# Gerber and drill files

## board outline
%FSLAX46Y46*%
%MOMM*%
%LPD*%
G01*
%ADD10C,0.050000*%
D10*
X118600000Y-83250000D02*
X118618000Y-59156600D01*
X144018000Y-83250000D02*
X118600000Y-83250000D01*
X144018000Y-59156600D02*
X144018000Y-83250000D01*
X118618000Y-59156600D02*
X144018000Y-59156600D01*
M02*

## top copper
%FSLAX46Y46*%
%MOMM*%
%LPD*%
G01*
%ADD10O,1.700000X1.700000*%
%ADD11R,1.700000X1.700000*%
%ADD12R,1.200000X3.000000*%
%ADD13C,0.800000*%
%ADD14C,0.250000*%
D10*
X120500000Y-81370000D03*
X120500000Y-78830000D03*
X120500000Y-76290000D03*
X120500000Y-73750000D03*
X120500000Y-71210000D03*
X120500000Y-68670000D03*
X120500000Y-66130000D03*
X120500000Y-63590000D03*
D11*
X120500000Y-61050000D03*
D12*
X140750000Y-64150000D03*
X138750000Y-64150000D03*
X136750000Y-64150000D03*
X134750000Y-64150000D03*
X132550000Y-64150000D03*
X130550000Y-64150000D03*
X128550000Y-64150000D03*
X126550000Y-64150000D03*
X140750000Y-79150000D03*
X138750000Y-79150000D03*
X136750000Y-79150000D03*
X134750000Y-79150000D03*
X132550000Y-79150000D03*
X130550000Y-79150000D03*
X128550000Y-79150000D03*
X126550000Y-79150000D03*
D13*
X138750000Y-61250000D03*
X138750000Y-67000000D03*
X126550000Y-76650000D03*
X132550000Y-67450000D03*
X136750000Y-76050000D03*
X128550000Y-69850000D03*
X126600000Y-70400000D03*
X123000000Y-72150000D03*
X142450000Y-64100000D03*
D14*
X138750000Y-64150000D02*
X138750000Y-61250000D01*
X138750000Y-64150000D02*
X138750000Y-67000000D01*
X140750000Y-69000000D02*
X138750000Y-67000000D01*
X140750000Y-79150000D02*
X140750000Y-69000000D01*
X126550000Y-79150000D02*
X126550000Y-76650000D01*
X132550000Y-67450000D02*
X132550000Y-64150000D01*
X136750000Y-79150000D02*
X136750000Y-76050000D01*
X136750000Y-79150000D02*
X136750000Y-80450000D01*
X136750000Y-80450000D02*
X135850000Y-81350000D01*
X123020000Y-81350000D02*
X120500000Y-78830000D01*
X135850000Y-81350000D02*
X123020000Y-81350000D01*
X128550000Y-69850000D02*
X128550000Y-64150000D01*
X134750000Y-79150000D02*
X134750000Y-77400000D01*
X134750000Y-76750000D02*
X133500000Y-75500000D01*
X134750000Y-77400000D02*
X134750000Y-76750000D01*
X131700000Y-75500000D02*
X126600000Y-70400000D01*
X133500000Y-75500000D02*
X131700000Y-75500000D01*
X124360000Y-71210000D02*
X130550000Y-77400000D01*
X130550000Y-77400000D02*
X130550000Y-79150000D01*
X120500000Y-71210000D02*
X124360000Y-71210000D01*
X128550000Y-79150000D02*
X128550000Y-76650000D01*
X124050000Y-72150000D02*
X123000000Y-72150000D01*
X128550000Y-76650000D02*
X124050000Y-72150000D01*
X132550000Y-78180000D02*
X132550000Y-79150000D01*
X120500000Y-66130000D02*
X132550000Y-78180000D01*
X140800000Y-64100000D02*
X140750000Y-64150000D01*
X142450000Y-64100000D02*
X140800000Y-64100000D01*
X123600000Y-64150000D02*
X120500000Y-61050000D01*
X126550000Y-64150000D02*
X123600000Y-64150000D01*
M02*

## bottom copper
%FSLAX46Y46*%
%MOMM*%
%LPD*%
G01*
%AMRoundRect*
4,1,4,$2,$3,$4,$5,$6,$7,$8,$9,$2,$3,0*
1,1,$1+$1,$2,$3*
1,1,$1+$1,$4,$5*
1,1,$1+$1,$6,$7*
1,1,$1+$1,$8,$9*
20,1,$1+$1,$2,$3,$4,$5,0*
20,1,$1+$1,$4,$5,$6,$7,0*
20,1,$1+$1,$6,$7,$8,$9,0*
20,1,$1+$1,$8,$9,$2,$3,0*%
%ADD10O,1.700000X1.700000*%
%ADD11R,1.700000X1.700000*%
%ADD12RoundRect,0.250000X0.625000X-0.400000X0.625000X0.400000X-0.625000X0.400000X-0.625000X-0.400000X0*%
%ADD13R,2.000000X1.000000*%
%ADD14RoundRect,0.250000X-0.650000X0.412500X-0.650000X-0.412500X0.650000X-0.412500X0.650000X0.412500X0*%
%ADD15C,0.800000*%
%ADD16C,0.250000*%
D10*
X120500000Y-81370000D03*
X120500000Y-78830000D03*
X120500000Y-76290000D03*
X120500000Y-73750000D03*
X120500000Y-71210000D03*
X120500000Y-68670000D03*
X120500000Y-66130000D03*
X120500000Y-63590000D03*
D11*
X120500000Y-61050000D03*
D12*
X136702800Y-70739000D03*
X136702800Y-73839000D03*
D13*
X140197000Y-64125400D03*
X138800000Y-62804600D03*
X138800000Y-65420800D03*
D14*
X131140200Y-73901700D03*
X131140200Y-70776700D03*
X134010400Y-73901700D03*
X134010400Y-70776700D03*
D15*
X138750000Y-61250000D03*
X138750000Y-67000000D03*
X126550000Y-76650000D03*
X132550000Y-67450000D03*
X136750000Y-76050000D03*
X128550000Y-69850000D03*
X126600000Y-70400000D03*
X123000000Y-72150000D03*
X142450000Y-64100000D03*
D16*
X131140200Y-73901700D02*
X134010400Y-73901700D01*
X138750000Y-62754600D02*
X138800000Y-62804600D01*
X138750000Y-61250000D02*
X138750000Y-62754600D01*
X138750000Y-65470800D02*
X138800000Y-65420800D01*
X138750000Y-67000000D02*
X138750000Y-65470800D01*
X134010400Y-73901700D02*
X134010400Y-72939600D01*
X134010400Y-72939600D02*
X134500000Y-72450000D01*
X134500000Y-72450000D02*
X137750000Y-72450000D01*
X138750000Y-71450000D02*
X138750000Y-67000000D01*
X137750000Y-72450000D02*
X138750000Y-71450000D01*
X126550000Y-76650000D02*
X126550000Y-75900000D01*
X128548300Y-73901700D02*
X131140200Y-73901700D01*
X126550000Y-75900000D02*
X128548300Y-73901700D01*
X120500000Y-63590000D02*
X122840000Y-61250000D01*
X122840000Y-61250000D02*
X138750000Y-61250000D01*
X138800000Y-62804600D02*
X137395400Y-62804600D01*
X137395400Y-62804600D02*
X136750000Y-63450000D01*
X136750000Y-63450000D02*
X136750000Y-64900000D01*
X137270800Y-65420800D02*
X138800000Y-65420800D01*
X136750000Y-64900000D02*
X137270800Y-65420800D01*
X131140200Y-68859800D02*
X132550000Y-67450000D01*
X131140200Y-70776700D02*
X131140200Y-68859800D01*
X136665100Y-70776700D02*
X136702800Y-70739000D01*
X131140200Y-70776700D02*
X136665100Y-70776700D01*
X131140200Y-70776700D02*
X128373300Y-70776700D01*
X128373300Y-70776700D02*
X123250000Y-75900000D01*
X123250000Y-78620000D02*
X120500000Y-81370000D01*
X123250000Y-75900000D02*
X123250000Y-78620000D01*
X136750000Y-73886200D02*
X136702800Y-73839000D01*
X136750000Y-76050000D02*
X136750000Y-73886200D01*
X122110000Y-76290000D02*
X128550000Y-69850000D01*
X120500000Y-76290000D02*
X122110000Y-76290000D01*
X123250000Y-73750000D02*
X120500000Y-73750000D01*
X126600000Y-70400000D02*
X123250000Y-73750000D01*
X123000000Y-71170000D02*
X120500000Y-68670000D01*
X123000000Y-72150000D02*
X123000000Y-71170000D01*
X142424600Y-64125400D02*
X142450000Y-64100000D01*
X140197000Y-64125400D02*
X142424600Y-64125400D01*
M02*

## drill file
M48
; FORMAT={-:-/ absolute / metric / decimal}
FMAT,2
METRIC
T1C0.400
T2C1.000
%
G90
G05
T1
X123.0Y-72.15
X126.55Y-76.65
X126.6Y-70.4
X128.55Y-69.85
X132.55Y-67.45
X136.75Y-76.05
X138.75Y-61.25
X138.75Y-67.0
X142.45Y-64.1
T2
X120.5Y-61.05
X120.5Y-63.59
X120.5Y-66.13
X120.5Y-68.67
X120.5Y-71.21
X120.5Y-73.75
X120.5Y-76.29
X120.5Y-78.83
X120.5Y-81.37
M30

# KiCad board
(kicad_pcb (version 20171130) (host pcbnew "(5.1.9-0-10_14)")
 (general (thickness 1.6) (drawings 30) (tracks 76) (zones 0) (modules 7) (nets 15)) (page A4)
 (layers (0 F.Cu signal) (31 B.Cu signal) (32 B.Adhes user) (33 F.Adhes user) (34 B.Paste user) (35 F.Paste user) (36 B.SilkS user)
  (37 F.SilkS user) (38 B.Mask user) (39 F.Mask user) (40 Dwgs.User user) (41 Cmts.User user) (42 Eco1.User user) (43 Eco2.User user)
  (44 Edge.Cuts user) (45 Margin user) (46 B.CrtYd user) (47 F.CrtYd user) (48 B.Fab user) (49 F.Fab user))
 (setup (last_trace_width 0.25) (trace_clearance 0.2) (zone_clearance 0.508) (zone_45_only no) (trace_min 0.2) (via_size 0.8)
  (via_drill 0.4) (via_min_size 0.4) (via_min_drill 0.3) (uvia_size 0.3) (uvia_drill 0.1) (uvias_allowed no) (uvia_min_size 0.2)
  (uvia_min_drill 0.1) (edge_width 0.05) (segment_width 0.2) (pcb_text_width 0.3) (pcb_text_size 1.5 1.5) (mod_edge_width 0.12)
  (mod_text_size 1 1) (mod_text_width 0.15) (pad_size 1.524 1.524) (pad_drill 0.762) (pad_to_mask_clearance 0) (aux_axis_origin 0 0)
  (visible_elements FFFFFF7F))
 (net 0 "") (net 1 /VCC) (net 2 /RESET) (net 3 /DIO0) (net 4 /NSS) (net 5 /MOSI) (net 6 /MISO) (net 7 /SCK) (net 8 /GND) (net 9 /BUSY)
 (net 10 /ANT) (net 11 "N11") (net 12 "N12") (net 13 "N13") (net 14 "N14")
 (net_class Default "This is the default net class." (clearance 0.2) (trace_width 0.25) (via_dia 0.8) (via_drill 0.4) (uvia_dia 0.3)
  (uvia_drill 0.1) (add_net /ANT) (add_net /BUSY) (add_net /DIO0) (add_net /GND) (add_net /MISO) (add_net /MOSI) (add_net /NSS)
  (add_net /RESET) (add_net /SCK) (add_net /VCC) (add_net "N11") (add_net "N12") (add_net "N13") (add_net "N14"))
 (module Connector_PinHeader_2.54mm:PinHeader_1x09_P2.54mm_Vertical (layer F.Cu) (at 120.5 61.05)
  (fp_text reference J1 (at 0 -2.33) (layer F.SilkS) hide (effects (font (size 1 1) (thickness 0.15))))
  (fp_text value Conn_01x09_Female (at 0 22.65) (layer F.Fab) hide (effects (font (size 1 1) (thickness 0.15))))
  (pad 9 thru_hole oval (at 0 20.32) (size 1.7 1.7) (drill 1) (layers *.Cu *.Mask) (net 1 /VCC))
  (pad 8 thru_hole oval (at 0 17.78) (size 1.7 1.7) (drill 1) (layers *.Cu *.Mask) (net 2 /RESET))
  (pad 7 thru_hole oval (at 0 15.24) (size 1.7 1.7) (drill 1) (layers *.Cu *.Mask) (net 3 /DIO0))
  (pad 6 thru_hole oval (at 0 12.7) (size 1.7 1.7) (drill 1) (layers *.Cu *.Mask) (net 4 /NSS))
  (pad 5 thru_hole oval (at 0 10.16) (size 1.7 1.7) (drill 1) (layers *.Cu *.Mask) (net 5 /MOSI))
  (pad 4 thru_hole oval (at 0 7.62) (size 1.7 1.7) (drill 1) (layers *.Cu *.Mask) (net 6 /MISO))
  (pad 3 thru_hole oval (at 0 5.08) (size 1.7 1.7) (drill 1) (layers *.Cu *.Mask) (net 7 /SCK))
  (pad 2 thru_hole oval (at 0 2.54) (size 1.7 1.7) (drill 1) (layers *.Cu *.Mask) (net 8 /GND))
  (pad 1 thru_hole rect (at 0 0) (size 1.7 1.7) (drill 1) (layers *.Cu *.Mask) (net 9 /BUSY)))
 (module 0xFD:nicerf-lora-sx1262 (layer F.Cu) (at 134.15 70.15 90)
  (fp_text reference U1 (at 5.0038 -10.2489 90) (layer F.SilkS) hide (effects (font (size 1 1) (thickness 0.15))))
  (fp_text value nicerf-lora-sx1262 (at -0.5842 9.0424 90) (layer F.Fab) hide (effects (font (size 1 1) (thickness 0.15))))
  (pad 9 smd rect (at 6 6.6 90) (size 3 1.2) (layers F.Cu F.Paste F.Mask) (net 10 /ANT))
  (pad 10 smd rect (at 6 4.6 90) (size 3 1.2) (layers F.Cu F.Paste F.Mask) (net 8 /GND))
  (pad 11 smd rect (at 6 2.6 90) (size 3 1.2) (layers F.Cu F.Paste F.Mask) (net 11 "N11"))
  (pad 12 smd rect (at 6 0.6 90) (size 3 1.2) (layers F.Cu F.Paste F.Mask) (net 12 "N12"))
  (pad 13 smd rect (at 6 -1.6 90) (size 3 1.2) (layers F.Cu F.Paste F.Mask) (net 1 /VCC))
  (pad 14 smd rect (at 6 -3.6 90) (size 3 1.2) (layers F.Cu F.Paste F.Mask) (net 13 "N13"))
  (pad 15 smd rect (at 6 -5.6 90) (size 3 1.2) (layers F.Cu F.Paste F.Mask) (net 3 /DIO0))
  (pad 16 smd rect (at 6 -7.6 90) (size 3 1.2) (layers F.Cu F.Paste F.Mask) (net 9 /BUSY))
  (pad 8 smd rect (at -9 6.6 90) (size 3 1.2) (layers F.Cu F.Paste F.Mask) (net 8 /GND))
  (pad 7 smd rect (at -9 4.6 90) (size 3 1.2) (layers F.Cu F.Paste F.Mask) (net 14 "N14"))
  (pad 6 smd rect (at -9 2.6 90) (size 3 1.2) (layers F.Cu F.Paste F.Mask) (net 2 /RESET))
  (pad 5 smd rect (at -9 0.6 90) (size 3 1.2) (layers F.Cu F.Paste F.Mask) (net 4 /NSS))
  (pad 4 smd rect (at -9 -1.6 90) (size 3 1.2) (layers F.Cu F.Paste F.Mask) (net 7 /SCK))
  (pad 3 smd rect (at -9 -3.6 90) (size 3 1.2) (layers F.Cu F.Paste F.Mask) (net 5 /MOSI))
  (pad 2 smd rect (at -9 -5.6 90) (size 3 1.2) (layers F.Cu F.Paste F.Mask) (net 6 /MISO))
  (pad 1 smd rect (at -9 -7.6 90) (size 3 1.2) (layers F.Cu F.Paste F.Mask) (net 8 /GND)))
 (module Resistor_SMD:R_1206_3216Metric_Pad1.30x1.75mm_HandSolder (layer B.Cu) (at 136.7028 72.289 90)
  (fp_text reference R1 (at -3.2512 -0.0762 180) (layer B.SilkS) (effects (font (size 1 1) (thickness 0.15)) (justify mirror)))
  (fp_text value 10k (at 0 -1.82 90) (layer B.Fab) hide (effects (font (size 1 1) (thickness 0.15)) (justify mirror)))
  (pad 2 smd roundrect (at 1.55 0 90) (size 1.3 1.75) (layers B.Cu B.Paste B.Mask) (roundrect_rratio 0.192308) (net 1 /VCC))
  (pad 1 smd roundrect (at -1.55 0 90) (size 1.3 1.75) (layers B.Cu B.Paste B.Mask) (roundrect_rratio 0.192308) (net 2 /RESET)))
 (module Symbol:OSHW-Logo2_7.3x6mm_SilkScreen (layer B.Cu) (at 132.9944 64.2366 180)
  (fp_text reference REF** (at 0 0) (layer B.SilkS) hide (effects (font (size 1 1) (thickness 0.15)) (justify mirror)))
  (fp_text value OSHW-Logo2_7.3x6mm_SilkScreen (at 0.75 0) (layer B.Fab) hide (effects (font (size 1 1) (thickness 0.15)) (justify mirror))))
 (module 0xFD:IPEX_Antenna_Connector (layer B.Cu) (at 138.8 64.1 90)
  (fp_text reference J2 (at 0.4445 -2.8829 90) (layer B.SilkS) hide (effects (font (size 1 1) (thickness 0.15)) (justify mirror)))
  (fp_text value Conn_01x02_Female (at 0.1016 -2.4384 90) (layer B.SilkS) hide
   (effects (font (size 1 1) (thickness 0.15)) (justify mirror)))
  (pad 2 smd rect (at -0.0254 1.397 180) (size 2 1) (layers B.Cu B.Paste B.Mask) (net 10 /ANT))
  (pad 1 smd rect (at 1.2954 0 90) (size 1 2) (layers B.Cu B.Paste B.Mask) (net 8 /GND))
  (pad 1 smd rect (at -1.3208 0 180) (size 2 1) (layers B.Cu B.Paste B.Mask) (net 8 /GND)))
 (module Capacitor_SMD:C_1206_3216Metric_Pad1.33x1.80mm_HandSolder (layer B.Cu) (at 131.1402 72.3392 270)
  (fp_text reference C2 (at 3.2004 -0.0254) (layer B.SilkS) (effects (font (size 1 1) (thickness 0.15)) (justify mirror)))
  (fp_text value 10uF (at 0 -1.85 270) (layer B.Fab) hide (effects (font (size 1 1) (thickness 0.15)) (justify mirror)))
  (pad 2 smd roundrect (at 1.5625 0 270) (size 1.325 1.8) (layers B.Cu B.Paste B.Mask) (roundrect_rratio 0.188679) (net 8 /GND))
  (pad 1 smd roundrect (at -1.5625 0 270) (size 1.325 1.8) (layers B.Cu B.Paste B.Mask) (roundrect_rratio 0.188679) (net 1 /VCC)))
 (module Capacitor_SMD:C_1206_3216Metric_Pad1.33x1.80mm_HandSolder (layer B.Cu) (at 134.0104 72.3392 270)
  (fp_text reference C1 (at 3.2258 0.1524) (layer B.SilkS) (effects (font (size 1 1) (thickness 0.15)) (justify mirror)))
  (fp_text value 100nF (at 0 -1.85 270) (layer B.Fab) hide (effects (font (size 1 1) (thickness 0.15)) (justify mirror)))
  (pad 2 smd roundrect (at 1.5625 0 270) (size 1.325 1.8) (layers B.Cu B.Paste B.Mask) (roundrect_rratio 0.188679) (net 8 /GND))
  (pad 1 smd roundrect (at -1.5625 0 270) (size 1.325 1.8) (layers B.Cu B.Paste B.Mask) (roundrect_rratio 0.188679) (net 1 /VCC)))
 (gr_line (start 118.6 83.25) (end 118.618 59.1566) (layer Edge.Cuts) (width 0.05))
 (gr_line (start 144.018 83.25) (end 118.6 83.25) (layer Edge.Cuts) (width 0.05))
 (gr_line (start 144.018 59.1566) (end 144.018 83.25) (layer Edge.Cuts) (width 0.05))
 (gr_line (start 118.618 59.1566) (end 144.018 59.1566) (layer Edge.Cuts) (width 0.05))
 (segment (start 131.1402 73.9017) (end 134.0104 73.9017) (width 0.25) (layer B.Cu) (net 8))
 (via (at 138.75 61.25) (size 0.8) (drill 0.4) (layers F.Cu B.Cu) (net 8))
 (segment (start 138.75 64.15) (end 138.75 61.25) (width 0.25) (layer F.Cu) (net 8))
 (segment (start 138.75 62.7546) (end 138.8 62.8046) (width 0.25) (layer B.Cu) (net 8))
 (segment (start 138.75 61.25) (end 138.75 62.7546) (width 0.25) (layer B.Cu) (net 8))
 (via (at 138.75 67) (size 0.8) (drill 0.4) (layers F.Cu B.Cu) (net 8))
 (segment (start 138.75 64.15) (end 138.75 67) (width 0.25) (layer F.Cu) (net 8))
 (segment (start 138.75 65.4708) (end 138.8 65.4208) (width 0.25) (layer B.Cu) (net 8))
 (segment (start 138.75 67) (end 138.75 65.4708) (width 0.25) (layer B.Cu) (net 8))
 (segment (start 134.0104 73.9017) (end 134.0104 72.9396) (width 0.25) (layer B.Cu) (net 8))
 (segment (start 134.0104 72.9396) (end 134.5 72.45) (width 0.25) (layer B.Cu) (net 8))
 (segment (start 134.5 72.45) (end 137.75 72.45) (width 0.25) (layer B.Cu) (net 8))
 (segment (start 138.75 71.45) (end 138.75 67) (width 0.25) (layer B.Cu) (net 8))
 (segment (start 137.75 72.45) (end 138.75 71.45) (width 0.25) (layer B.Cu) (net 8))
 (segment (start 140.75 69) (end 138.75 67) (width 0.25) (layer F.Cu) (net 8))
 (segment (start 140.75 79.15) (end 140.75 69) (width 0.25) (layer F.Cu) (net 8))
 (via (at 126.55 76.65) (size 0.8) (drill 0.4) (layers F.Cu B.Cu) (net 8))
 (segment (start 126.55 79.15) (end 126.55 76.65) (width 0.25) (layer F.Cu) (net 8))
 (segment (start 126.55 76.65) (end 126.55 75.9) (width 0.25) (layer B.Cu) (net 8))
 (segment (start 128.5483 73.9017) (end 131.1402 73.9017) (width 0.25) (layer B.Cu) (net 8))
 (segment (start 126.55 75.9) (end 128.5483 73.9017) (width 0.25) (layer B.Cu) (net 8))
 (segment (start 120.5 63.59) (end 122.84 61.25) (width 0.25) (layer B.Cu) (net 8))
 (segment (start 122.84 61.25) (end 138.75 61.25) (width 0.25) (layer B.Cu) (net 8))
 (segment (start 138.8 62.8046) (end 137.3954 62.8046) (width 0.25) (layer B.Cu) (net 8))
 (segment (start 137.3954 62.8046) (end 136.75 63.45) (width 0.25) (layer B.Cu) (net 8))
 (segment (start 136.75 63.45) (end 136.75 64.9) (width 0.25) (layer B.Cu) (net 8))
 (segment (start 137.2708 65.4208) (end 138.8 65.4208) (width 0.25) (layer B.Cu) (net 8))
 (segment (start 136.75 64.9) (end 137.2708 65.4208) (width 0.25) (layer B.Cu) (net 8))
 (segment (start 131.1402 68.8598) (end 132.55 67.45) (width 0.25) (layer B.Cu) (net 1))
 (via (at 132.55 67.45) (size 0.8) (drill 0.4) (layers F.Cu B.Cu) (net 1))
 (segment (start 131.1402 70.7767) (end 131.1402 68.8598) (width 0.25) (layer B.Cu) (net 1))
 (segment (start 132.55 67.45) (end 132.55 64.15) (width 0.25) (layer F.Cu) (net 1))
 (segment (start 136.6651 70.7767) (end 136.7028 70.739) (width 0.25) (layer B.Cu) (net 1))
 (segment (start 131.1402 70.7767) (end 136.6651 70.7767) (width 0.25) (layer B.Cu) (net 1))
 (segment (start 131.1402 70.7767) (end 128.3733 70.7767) (width 0.25) (layer B.Cu) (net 1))
 (segment (start 128.3733 70.7767) (end 123.25 75.9) (width 0.25) (layer B.Cu) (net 1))
 (segment (start 123.25 78.62) (end 120.5 81.37) (width 0.25) (layer B.Cu) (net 1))
 (segment (start 123.25 75.9) (end 123.25 78.62) (width 0.25) (layer B.Cu) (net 1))
 (via (at 136.75 76.05) (size 0.8) (drill 0.4) (layers F.Cu B.Cu) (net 2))
 (segment (start 136.75 79.15) (end 136.75 76.05) (width 0.25) (layer F.Cu) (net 2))
 (segment (start 136.75 73.8862) (end 136.7028 73.839) (width 0.25) (layer B.Cu) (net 2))
 (segment (start 136.75 76.05) (end 136.75 73.8862) (width 0.25) (layer B.Cu) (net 2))
 (segment (start 136.75 79.15) (end 136.75 80.45) (width 0.25) (layer F.Cu) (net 2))
 (segment (start 136.75 80.45) (end 135.85 81.35) (width 0.25) (layer F.Cu) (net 2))
 (segment (start 123.02 81.35) (end 120.5 78.83) (width 0.25) (layer F.Cu) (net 2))
 (segment (start 135.85 81.35) (end 123.02 81.35) (width 0.25) (layer F.Cu) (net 2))
 (via (at 128.55 69.85) (size 0.8) (drill 0.4) (layers F.Cu B.Cu) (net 3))
 (segment (start 122.11 76.29) (end 128.55 69.85) (width 0.25) (layer B.Cu) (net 3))
 (segment (start 120.5 76.29) (end 122.11 76.29) (width 0.25) (layer B.Cu) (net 3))
 (segment (start 128.55 69.85) (end 128.55 64.15) (width 0.25) (layer F.Cu) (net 3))
 (segment (start 134.75 79.15) (end 134.75 77.4) (width 0.25) (layer F.Cu) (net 4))
 (segment (start 134.75 76.75) (end 133.5 75.5) (width 0.25) (layer F.Cu) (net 4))
 (segment (start 134.75 77.4) (end 134.75 76.75) (width 0.25) (layer F.Cu) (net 4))
 (via (at 126.6 70.4) (size 0.8) (drill 0.4) (layers F.Cu B.Cu) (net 4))
 (segment (start 131.7 75.5) (end 126.6 70.4) (width 0.25) (layer F.Cu) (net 4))
 (segment (start 133.5 75.5) (end 131.7 75.5) (width 0.25) (layer F.Cu) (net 4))
 (segment (start 123.25 73.75) (end 120.5 73.75) (width 0.25) (layer B.Cu) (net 4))
 (segment (start 126.6 70.4) (end 123.25 73.75) (width 0.25) (layer B.Cu) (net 4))
 (segment (start 124.36 71.21) (end 130.55 77.4) (width 0.25) (layer F.Cu) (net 5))
 (segment (start 130.55 77.4) (end 130.55 79.15) (width 0.25) (layer F.Cu) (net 5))
 (segment (start 120.5 71.21) (end 124.36 71.21) (width 0.25) (layer F.Cu) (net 5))
 (segment (start 128.55 79.15) (end 128.55 76.65) (width 0.25) (layer F.Cu) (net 6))
 (via (at 123 72.15) (size 0.8) (drill 0.4) (layers F.Cu B.Cu) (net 6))
 (segment (start 124.05 72.15) (end 123 72.15) (width 0.25) (layer F.Cu) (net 6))
 (segment (start 128.55 76.65) (end 124.05 72.15) (width 0.25) (layer F.Cu) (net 6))
 (segment (start 123 71.17) (end 120.5 68.67) (width 0.25) (layer B.Cu) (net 6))
 (segment (start 123 72.15) (end 123 71.17) (width 0.25) (layer B.Cu) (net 6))
 (segment (start 132.55 78.18) (end 132.55 79.15) (width 0.25) (layer F.Cu) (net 7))
 (segment (start 120.5 66.13) (end 132.55 78.18) (width 0.25) (layer F.Cu) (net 7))
 (via (at 142.45 64.1) (size 0.8) (drill 0.4) (layers F.Cu B.Cu) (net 10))
 (segment (start 142.4246 64.1254) (end 142.45 64.1) (width 0.25) (layer B.Cu) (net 10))
 (segment (start 140.197 64.1254) (end 142.4246 64.1254) (width 0.25) (layer B.Cu) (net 10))
 (segment (start 140.8 64.1) (end 140.75 64.15) (width 0.25) (layer F.Cu) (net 10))
 (segment (start 142.45 64.1) (end 140.8 64.1) (width 0.25) (layer F.Cu) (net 10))
 (segment (start 123.6 64.15) (end 120.5 61.05) (width 0.25) (layer F.Cu) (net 9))
 (segment (start 126.55 64.15) (end 123.6 64.15) (width 0.25) (layer F.Cu) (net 9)))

